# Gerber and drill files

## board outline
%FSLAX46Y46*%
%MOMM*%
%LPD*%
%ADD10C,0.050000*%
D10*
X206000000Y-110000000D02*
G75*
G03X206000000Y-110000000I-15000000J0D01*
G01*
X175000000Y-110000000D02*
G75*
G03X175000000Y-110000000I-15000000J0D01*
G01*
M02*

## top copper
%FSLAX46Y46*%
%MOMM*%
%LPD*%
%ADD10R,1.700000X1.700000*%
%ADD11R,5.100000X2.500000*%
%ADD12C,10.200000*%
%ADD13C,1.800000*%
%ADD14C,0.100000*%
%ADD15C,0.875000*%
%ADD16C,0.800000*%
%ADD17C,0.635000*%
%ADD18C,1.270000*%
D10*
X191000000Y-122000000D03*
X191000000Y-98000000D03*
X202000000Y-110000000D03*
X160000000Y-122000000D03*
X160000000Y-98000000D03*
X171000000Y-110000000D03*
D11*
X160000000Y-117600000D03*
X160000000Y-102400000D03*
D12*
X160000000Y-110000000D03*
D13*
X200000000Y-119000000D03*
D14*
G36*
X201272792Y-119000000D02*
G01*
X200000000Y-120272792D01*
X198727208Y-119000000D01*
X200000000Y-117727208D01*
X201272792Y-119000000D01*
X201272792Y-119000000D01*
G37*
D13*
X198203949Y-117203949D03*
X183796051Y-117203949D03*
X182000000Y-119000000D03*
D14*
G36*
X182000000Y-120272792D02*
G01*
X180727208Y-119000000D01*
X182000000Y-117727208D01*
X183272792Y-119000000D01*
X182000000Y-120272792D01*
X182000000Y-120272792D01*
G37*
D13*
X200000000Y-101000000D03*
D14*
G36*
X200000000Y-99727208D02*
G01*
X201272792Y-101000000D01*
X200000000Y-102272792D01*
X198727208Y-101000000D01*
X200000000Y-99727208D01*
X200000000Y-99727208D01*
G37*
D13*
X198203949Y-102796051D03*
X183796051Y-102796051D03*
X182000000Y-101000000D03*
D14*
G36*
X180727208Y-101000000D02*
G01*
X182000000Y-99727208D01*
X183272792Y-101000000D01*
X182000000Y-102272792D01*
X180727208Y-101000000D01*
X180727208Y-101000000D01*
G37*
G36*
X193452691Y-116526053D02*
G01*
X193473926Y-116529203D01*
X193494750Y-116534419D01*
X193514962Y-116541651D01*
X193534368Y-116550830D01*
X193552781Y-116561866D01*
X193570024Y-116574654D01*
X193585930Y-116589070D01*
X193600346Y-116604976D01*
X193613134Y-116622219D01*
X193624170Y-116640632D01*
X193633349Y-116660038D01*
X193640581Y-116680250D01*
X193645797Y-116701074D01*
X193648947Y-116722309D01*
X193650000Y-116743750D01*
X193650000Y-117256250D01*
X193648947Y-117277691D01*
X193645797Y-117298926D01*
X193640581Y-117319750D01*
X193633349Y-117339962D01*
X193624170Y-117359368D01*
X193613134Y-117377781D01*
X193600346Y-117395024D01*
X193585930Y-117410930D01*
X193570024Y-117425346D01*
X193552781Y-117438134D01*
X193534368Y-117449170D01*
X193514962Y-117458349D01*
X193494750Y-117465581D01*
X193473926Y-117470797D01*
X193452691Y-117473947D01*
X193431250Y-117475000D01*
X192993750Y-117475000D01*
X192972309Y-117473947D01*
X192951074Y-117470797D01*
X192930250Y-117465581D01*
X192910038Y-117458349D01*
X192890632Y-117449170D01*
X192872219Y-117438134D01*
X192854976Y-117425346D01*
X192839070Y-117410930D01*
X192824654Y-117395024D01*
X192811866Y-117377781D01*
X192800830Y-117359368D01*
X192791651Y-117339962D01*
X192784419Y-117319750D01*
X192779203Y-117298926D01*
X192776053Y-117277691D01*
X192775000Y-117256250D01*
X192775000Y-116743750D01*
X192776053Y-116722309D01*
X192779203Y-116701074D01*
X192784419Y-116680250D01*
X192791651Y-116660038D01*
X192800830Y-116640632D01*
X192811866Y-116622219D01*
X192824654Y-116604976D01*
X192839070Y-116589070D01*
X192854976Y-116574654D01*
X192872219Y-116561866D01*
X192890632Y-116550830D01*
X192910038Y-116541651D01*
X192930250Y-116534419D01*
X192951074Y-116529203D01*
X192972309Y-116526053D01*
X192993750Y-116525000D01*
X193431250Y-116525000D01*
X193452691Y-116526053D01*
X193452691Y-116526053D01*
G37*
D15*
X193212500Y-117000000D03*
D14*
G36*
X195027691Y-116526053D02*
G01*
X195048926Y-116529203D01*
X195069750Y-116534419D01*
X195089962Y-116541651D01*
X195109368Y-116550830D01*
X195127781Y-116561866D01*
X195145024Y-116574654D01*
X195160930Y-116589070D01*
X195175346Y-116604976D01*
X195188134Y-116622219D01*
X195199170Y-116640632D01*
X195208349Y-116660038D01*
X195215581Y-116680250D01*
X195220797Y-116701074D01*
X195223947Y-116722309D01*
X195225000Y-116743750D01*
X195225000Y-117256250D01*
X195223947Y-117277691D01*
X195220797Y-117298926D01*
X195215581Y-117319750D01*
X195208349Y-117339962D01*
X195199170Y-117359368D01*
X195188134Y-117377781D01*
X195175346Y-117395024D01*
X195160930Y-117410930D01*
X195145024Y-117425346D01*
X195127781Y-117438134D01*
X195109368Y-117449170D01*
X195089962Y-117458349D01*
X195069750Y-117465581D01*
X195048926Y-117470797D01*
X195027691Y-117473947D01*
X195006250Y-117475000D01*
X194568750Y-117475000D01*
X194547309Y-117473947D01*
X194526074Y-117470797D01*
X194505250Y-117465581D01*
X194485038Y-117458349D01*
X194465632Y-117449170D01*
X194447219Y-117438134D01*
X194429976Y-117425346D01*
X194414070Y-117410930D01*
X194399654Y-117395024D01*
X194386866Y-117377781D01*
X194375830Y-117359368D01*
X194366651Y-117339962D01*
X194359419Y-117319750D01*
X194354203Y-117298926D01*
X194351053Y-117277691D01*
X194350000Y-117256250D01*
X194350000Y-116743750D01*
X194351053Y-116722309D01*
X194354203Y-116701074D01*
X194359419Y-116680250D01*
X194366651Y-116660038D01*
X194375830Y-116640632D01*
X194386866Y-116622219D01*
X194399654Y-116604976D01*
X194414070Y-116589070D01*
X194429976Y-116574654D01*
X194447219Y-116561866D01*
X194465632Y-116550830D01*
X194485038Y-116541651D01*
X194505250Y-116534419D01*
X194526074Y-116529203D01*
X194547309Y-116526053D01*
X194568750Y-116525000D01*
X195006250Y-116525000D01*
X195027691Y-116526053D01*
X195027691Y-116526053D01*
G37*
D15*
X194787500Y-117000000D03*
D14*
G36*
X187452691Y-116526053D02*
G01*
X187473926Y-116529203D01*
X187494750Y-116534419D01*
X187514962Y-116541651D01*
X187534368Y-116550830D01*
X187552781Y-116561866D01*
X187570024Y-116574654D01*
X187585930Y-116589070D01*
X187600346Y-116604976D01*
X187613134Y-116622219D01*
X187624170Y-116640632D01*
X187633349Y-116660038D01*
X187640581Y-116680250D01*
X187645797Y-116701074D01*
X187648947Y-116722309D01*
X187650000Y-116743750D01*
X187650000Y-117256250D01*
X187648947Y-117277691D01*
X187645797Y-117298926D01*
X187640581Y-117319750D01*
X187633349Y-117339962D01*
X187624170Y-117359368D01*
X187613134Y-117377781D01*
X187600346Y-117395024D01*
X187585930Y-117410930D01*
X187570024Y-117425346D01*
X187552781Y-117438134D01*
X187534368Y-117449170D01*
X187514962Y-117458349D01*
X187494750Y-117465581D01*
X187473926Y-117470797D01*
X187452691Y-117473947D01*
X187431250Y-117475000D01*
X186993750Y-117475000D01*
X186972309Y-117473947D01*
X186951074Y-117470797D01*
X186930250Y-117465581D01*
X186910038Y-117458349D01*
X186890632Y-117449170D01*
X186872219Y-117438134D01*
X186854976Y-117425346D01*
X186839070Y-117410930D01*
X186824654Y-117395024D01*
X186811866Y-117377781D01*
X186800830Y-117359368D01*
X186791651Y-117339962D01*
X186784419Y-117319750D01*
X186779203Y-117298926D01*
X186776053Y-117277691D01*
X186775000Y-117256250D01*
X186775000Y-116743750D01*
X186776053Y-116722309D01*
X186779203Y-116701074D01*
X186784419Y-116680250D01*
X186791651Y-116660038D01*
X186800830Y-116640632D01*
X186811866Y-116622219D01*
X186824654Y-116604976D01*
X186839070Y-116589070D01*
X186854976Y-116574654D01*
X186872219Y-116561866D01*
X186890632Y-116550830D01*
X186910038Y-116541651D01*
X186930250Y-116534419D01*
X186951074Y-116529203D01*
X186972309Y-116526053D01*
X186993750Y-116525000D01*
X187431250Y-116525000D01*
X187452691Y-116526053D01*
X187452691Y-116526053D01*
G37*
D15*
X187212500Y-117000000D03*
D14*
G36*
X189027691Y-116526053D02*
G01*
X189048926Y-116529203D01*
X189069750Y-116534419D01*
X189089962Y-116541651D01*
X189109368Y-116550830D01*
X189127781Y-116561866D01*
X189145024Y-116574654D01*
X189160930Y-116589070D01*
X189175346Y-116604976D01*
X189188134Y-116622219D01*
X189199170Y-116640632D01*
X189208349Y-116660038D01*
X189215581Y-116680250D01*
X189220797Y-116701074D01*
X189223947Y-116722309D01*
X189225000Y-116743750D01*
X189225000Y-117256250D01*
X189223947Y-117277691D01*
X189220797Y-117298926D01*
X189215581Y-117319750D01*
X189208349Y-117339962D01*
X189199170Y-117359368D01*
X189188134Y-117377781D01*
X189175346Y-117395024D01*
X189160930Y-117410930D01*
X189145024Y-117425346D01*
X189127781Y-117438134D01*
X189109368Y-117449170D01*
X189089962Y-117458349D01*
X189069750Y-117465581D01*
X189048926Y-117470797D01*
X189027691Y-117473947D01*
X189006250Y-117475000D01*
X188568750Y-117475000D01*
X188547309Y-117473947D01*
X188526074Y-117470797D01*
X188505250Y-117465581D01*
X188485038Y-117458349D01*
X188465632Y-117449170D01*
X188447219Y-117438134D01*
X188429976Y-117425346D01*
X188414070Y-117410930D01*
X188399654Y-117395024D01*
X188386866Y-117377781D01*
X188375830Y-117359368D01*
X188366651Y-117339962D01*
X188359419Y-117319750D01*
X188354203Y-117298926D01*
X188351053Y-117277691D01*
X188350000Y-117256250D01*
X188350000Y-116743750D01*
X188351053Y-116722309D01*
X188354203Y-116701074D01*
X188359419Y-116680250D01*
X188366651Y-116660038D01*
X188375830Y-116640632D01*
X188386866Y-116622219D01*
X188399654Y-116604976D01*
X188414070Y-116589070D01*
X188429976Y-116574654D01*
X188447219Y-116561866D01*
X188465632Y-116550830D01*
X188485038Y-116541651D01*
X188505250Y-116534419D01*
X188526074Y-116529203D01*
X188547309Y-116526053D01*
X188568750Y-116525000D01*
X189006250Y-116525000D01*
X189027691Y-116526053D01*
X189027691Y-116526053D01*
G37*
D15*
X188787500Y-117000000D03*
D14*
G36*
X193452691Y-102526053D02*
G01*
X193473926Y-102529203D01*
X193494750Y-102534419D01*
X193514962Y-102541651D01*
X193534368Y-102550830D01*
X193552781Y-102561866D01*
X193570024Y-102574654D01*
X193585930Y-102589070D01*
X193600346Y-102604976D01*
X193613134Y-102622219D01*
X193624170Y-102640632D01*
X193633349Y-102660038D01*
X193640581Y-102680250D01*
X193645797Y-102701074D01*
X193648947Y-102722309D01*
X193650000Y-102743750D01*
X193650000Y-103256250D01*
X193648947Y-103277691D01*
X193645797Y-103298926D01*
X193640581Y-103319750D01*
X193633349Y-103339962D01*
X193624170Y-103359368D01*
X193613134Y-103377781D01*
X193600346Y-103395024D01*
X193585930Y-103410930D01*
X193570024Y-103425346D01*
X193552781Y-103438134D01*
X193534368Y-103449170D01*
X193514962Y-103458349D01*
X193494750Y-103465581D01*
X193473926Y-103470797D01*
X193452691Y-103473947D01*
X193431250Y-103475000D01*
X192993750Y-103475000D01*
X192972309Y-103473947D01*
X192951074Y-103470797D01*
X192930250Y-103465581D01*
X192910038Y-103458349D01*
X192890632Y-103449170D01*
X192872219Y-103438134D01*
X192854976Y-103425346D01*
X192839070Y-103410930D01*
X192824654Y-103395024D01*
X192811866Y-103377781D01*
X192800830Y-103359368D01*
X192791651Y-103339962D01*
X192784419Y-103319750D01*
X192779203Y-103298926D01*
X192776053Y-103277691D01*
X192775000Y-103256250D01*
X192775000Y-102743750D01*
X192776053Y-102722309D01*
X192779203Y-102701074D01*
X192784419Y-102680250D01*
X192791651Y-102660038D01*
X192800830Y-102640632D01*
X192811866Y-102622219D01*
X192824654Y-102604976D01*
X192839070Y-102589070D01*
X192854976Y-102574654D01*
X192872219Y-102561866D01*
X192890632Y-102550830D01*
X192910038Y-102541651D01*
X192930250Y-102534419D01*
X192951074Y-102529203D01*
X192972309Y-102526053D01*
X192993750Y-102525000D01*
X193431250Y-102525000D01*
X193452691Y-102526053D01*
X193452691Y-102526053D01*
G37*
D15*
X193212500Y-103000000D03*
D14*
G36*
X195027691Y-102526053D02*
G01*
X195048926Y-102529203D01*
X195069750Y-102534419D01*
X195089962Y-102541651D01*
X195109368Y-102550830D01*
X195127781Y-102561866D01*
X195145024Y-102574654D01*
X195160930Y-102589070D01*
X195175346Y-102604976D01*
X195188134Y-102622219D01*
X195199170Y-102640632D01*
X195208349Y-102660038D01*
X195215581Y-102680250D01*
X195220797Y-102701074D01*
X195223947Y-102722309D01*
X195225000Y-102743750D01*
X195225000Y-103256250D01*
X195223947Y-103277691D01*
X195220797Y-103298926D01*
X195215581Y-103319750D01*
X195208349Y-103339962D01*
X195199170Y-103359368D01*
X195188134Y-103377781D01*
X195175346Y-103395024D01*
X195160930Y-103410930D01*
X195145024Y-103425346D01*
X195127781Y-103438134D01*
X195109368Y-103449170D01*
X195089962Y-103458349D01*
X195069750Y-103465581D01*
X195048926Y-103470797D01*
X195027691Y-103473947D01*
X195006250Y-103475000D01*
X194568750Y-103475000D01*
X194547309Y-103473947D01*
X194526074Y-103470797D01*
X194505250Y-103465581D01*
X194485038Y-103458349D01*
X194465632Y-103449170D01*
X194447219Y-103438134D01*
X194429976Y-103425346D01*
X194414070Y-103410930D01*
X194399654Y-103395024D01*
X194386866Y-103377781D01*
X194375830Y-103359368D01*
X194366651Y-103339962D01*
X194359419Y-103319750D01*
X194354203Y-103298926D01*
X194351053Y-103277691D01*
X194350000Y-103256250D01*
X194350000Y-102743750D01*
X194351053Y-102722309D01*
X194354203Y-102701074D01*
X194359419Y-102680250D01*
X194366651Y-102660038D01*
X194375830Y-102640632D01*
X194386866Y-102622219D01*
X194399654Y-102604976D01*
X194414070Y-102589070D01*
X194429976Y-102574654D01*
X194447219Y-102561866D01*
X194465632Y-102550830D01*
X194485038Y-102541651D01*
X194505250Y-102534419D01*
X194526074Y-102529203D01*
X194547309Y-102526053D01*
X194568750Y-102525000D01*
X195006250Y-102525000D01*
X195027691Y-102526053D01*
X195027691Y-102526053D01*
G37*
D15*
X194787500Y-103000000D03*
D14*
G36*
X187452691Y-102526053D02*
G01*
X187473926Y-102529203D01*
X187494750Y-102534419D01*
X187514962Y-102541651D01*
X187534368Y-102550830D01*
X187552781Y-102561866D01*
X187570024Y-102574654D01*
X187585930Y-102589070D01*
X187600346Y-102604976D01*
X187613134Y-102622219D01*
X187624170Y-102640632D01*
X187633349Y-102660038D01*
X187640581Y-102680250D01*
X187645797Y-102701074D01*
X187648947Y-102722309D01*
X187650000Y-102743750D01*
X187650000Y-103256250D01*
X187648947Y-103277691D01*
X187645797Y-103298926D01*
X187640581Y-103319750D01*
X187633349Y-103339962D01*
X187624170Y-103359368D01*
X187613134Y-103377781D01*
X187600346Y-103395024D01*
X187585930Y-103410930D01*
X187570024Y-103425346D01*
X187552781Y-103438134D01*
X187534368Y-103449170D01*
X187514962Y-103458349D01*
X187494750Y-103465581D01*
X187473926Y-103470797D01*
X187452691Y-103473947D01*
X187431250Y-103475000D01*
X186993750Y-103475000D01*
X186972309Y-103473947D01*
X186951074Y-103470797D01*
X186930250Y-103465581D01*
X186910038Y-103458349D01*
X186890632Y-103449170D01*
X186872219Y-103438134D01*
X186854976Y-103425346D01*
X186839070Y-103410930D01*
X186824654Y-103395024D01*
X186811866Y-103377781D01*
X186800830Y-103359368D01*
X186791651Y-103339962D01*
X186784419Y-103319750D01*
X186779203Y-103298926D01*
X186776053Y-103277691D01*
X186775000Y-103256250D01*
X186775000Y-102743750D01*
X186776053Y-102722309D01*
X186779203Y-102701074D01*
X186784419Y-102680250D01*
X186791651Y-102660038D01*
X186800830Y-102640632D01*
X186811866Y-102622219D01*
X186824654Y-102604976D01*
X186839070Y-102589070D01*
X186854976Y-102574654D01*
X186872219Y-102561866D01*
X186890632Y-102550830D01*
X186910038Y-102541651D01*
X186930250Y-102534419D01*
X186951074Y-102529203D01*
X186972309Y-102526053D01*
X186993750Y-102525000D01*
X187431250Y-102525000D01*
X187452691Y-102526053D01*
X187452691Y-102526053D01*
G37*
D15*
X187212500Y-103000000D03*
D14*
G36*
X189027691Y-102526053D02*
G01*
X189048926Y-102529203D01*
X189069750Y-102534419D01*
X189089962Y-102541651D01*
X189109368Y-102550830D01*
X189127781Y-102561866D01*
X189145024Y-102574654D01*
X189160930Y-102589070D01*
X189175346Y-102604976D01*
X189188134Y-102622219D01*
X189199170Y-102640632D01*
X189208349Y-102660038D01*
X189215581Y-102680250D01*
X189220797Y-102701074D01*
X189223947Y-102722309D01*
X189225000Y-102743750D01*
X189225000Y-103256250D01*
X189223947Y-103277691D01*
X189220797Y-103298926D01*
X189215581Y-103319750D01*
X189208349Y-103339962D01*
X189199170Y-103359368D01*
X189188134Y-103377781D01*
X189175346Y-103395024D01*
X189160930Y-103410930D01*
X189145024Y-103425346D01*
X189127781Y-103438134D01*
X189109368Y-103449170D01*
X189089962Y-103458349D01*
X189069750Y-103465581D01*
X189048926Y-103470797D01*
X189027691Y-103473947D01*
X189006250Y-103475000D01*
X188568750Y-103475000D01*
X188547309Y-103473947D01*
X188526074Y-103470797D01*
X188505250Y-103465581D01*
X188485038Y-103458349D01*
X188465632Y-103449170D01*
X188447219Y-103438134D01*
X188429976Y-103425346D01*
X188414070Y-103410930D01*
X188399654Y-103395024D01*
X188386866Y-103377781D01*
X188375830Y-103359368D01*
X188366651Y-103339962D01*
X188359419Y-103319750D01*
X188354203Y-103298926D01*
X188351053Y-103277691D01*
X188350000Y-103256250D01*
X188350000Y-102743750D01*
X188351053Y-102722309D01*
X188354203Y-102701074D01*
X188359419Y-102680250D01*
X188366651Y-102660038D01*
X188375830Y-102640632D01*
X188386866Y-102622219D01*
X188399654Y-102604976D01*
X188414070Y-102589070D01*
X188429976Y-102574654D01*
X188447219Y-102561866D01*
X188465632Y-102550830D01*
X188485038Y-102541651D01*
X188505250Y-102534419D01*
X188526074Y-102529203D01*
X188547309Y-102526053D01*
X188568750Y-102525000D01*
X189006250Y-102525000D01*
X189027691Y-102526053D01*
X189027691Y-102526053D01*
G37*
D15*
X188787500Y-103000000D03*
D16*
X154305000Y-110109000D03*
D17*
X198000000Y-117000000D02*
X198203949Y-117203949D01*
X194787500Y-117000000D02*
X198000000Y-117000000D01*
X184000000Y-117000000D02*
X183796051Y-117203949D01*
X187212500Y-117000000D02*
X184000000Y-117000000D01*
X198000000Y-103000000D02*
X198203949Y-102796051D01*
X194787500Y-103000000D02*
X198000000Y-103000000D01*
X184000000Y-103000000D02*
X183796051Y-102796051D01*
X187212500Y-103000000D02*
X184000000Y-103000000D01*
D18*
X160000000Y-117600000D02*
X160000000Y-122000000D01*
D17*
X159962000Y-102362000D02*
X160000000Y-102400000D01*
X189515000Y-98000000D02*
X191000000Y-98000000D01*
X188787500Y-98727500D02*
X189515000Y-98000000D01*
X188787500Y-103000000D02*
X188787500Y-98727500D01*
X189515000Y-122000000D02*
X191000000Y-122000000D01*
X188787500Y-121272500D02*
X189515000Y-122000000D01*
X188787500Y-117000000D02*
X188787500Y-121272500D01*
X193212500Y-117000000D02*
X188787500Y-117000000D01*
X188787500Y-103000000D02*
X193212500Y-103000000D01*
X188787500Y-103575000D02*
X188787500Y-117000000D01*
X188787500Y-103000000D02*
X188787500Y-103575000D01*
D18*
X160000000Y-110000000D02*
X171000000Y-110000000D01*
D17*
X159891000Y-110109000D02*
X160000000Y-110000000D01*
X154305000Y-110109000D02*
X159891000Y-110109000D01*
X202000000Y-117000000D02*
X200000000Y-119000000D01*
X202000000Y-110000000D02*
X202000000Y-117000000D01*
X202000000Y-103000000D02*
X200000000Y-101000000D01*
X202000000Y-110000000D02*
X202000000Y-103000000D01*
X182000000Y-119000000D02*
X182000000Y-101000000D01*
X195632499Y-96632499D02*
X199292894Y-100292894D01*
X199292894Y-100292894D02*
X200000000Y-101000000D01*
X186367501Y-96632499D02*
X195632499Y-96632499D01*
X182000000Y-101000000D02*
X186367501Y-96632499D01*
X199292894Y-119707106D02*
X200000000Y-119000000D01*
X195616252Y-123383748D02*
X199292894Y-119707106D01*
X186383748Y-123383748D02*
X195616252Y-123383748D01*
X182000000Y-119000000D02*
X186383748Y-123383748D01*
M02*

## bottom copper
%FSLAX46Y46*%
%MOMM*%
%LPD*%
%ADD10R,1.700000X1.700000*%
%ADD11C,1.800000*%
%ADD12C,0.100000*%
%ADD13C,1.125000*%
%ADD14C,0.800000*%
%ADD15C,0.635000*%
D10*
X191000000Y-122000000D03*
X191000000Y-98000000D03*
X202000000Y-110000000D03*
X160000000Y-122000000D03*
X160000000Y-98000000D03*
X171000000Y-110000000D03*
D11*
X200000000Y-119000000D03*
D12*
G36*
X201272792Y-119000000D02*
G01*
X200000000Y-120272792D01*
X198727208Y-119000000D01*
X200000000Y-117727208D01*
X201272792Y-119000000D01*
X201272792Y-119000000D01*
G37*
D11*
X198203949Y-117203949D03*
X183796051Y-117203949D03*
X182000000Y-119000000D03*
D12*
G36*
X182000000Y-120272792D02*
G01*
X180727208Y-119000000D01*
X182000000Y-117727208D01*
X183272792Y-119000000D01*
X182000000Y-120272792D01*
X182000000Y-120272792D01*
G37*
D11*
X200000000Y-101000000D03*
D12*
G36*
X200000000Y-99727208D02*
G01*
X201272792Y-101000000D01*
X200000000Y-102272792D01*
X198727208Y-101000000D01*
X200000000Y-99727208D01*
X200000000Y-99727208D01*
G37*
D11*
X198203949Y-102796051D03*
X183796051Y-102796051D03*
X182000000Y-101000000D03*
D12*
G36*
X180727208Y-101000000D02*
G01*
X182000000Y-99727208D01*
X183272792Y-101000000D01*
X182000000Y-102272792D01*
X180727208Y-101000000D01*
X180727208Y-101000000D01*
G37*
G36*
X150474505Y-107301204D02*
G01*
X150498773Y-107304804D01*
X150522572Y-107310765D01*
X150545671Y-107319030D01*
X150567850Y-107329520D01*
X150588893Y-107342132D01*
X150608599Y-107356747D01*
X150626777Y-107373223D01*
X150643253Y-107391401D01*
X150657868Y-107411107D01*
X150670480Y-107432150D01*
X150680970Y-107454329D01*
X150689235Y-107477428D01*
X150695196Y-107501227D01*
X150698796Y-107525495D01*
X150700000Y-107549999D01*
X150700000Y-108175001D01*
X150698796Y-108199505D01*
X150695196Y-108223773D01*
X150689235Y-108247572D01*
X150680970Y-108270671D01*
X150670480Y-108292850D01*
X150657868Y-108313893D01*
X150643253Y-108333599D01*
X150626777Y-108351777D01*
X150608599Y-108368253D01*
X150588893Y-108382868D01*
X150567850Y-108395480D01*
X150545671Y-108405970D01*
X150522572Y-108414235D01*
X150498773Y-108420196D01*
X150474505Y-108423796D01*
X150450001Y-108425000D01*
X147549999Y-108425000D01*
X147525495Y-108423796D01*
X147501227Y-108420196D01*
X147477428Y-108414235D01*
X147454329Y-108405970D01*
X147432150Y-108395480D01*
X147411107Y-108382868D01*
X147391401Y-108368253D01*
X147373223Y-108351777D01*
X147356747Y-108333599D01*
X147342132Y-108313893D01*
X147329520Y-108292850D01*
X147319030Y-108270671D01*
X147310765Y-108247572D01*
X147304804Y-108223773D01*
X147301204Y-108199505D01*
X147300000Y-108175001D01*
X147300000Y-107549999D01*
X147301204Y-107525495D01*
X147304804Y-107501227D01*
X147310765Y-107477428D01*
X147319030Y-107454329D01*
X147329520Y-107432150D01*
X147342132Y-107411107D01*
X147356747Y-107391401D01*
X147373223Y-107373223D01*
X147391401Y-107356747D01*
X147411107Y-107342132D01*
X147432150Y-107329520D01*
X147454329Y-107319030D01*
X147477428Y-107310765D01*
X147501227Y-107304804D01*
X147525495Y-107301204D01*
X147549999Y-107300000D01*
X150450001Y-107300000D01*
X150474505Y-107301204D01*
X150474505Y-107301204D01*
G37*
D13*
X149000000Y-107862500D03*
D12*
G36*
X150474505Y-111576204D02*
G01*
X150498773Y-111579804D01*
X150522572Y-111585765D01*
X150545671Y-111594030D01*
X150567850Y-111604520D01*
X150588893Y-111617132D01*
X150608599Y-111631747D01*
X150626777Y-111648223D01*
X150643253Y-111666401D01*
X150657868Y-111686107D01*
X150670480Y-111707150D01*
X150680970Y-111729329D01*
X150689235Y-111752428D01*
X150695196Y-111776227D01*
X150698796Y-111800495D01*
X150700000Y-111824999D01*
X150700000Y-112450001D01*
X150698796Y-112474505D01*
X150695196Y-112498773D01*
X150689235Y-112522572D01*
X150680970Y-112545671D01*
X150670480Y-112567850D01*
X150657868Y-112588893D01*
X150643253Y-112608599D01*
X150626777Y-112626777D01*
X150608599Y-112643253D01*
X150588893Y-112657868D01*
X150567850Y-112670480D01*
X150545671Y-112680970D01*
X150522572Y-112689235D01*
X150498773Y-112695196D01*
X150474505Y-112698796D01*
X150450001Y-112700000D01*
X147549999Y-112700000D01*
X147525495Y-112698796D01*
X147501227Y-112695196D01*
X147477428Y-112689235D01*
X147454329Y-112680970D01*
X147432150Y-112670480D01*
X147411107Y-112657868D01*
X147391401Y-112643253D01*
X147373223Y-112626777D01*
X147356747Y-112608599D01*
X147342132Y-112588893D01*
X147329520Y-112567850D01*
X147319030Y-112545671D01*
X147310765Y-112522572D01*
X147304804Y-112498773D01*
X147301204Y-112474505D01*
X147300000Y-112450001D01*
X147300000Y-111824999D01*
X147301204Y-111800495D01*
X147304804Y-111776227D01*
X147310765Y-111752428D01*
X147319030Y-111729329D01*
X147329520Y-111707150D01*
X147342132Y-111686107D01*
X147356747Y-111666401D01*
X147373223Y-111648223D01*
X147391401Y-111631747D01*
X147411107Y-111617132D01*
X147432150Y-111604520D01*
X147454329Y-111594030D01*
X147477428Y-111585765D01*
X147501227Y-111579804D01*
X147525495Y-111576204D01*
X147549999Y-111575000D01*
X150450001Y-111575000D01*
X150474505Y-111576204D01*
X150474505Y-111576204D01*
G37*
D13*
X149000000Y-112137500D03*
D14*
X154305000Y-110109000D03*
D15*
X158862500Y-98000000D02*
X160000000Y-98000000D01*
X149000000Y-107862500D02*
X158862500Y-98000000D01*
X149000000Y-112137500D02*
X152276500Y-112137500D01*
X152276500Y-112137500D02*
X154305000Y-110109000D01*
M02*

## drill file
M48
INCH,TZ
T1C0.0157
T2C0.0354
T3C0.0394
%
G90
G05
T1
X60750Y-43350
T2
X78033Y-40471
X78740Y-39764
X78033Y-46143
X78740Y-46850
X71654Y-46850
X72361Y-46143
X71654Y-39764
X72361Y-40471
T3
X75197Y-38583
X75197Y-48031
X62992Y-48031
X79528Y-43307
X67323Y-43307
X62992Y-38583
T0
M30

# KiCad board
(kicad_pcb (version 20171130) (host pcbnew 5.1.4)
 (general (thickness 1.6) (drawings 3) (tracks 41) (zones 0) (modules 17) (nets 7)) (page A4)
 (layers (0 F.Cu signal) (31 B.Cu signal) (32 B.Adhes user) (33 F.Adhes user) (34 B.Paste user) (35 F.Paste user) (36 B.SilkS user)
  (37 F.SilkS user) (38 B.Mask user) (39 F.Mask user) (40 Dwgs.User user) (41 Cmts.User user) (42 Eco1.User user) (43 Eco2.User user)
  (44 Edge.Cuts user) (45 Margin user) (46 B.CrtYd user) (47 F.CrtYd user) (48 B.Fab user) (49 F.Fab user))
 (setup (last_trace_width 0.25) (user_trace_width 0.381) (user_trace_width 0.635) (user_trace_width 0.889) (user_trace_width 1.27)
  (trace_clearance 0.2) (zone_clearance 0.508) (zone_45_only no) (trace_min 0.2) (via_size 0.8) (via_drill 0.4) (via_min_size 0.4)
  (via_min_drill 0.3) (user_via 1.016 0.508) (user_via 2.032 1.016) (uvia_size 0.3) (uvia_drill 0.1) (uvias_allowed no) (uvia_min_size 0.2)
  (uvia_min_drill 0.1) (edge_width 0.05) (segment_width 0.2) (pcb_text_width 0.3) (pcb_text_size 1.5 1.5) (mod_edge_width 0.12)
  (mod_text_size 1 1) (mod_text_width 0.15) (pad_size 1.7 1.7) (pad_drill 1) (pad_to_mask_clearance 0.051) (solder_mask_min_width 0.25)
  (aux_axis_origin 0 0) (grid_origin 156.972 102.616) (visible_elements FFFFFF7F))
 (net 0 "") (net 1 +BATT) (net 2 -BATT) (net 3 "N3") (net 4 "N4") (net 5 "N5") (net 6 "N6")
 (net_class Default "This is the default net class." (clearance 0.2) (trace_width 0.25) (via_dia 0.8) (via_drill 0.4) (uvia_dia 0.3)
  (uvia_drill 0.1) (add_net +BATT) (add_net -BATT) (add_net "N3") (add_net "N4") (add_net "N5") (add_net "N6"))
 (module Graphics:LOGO (layer B.Cu) (at 184.785 116.205)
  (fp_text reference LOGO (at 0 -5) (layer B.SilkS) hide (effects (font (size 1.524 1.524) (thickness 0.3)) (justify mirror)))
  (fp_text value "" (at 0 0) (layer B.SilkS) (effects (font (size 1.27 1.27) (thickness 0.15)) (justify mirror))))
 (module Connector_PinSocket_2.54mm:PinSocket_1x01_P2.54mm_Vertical (layer F.Cu) (at 191 122)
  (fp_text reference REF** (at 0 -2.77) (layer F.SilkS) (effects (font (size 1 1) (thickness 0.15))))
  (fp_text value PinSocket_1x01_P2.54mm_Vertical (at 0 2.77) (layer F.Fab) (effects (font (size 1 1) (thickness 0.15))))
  (pad 1 thru_hole rect (at 0 0) (size 1.7 1.7) (drill 1) (layers *.Cu *.Mask) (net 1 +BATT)))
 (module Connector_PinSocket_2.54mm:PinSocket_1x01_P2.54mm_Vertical (layer F.Cu) (at 191 98)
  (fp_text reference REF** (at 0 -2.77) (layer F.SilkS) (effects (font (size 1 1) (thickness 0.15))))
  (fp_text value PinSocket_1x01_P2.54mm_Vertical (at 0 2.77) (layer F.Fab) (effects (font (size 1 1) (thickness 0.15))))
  (pad 1 thru_hole rect (at 0 0) (size 1.7 1.7) (drill 1) (layers *.Cu *.Mask) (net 1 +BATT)))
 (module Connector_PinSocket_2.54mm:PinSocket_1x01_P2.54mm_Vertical (layer F.Cu) (at 202 110)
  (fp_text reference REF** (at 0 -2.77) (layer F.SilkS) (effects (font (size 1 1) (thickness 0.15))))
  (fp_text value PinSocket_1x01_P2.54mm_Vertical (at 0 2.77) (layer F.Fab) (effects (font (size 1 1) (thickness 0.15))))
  (pad 1 thru_hole rect (at 0 0) (size 1.7 1.7) (drill 1) (layers *.Cu *.Mask) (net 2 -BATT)))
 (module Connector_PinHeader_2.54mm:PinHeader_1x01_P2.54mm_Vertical (layer F.Cu) (at 160 122 180)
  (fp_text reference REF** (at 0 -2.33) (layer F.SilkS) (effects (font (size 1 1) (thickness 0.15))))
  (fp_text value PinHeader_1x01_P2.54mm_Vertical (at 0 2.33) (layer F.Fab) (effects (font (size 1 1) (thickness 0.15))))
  (pad 1 thru_hole rect (at 0 0 180) (size 1.7 1.7) (drill 1) (layers *.Cu *.Mask) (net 1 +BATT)))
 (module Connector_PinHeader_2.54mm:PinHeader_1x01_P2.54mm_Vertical (layer F.Cu) (at 160 98)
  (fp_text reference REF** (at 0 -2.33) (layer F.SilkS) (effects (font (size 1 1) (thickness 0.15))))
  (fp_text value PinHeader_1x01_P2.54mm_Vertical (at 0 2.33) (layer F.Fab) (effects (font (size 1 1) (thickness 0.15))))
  (pad 1 thru_hole rect (at 0 0) (size 1.7 1.7) (drill 1) (layers *.Cu *.Mask) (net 1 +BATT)))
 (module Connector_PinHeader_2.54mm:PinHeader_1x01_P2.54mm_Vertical (layer F.Cu) (at 171 110 90)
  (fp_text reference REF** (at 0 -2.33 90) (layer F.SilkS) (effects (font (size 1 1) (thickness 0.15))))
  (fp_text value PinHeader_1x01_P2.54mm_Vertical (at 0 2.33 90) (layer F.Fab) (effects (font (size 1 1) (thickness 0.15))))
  (pad 1 thru_hole rect (at 0 0 90) (size 1.7 1.7) (drill 1) (layers *.Cu *.Mask) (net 2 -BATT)))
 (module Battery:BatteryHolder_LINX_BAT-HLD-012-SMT (layer F.Cu) (at 160 110 90)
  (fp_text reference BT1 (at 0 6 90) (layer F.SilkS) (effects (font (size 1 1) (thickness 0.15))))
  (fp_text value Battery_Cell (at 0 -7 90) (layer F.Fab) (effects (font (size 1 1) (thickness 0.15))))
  (pad 1 smd rect (at -7.6 0 90) (size 2.5 5.1) (layers F.Cu F.Paste F.Mask) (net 1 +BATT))
  (pad 1 smd rect (at 7.6 0 90) (size 2.5 5.1) (layers F.Cu F.Paste F.Mask) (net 1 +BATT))
  (pad 2 smd circle (at 0 0 90) (size 10.2 10.2) (layers F.Cu F.Paste F.Mask) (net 2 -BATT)))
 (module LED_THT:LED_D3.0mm (layer F.Cu) (at 200 119 135)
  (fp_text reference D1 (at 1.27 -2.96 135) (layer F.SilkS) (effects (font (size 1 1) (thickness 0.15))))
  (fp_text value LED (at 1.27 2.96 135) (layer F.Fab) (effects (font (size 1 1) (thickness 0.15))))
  (pad 1 thru_hole rect (at 0 0 135) (size 1.8 1.8) (drill 0.9) (layers *.Cu *.Mask) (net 2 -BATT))
  (pad 2 thru_hole circle (at 2.54 0 135) (size 1.8 1.8) (drill 0.9) (layers *.Cu *.Mask) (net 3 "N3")))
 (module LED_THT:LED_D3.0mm (layer F.Cu) (at 182 119 45)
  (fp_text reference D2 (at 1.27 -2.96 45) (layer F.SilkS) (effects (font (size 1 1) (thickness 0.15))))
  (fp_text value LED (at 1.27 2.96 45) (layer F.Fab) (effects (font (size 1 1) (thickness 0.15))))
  (pad 2 thru_hole circle (at 2.54 0 45) (size 1.8 1.8) (drill 0.9) (layers *.Cu *.Mask) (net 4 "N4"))
  (pad 1 thru_hole rect (at 0 0 45) (size 1.8 1.8) (drill 0.9) (layers *.Cu *.Mask) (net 2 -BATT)))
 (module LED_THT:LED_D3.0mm (layer F.Cu) (at 200 101 225)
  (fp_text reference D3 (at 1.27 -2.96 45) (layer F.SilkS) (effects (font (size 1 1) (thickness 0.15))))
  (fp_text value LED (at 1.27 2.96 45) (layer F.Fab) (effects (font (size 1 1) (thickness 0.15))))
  (pad 1 thru_hole rect (at 0 0 225) (size 1.8 1.8) (drill 0.9) (layers *.Cu *.Mask) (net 2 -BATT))
  (pad 2 thru_hole circle (at 2.54 0 225) (size 1.8 1.8) (drill 0.9) (layers *.Cu *.Mask) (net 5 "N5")))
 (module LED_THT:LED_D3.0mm (layer F.Cu) (at 182 101 315)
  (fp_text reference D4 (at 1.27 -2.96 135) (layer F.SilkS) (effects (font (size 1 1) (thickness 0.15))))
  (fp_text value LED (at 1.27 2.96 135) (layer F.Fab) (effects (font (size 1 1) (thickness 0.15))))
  (pad 2 thru_hole circle (at 2.54 0 315) (size 1.8 1.8) (drill 0.9) (layers *.Cu *.Mask) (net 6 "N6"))
  (pad 1 thru_hole rect (at 0 0 315) (size 1.8 1.8) (drill 0.9) (layers *.Cu *.Mask) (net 2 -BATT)))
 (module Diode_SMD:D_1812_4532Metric (layer B.Cu) (at 149 110 270)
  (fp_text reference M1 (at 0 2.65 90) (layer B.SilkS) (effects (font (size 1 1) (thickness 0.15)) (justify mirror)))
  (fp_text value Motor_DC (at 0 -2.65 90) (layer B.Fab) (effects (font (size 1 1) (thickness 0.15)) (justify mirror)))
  (pad 1 smd roundrect (at -2.1375 0 270) (size 1.125 3.4) (layers B.Cu B.Paste B.Mask) (roundrect_rratio 0.222222) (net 1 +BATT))
  (pad 2 smd roundrect (at 2.1375 0 270) (size 1.125 3.4) (layers B.Cu B.Paste B.Mask) (roundrect_rratio 0.222222) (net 2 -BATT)))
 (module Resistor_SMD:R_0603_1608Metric (layer F.Cu) (at 194 117)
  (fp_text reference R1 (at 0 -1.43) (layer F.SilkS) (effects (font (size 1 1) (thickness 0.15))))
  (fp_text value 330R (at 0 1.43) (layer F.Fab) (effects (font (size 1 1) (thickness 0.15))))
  (pad 1 smd roundrect (at -0.7875 0) (size 0.875 0.95) (layers F.Cu F.Paste F.Mask) (roundrect_rratio 0.25) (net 1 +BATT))
  (pad 2 smd roundrect (at 0.7875 0) (size 0.875 0.95) (layers F.Cu F.Paste F.Mask) (roundrect_rratio 0.25) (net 3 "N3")))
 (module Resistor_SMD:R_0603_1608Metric (layer F.Cu) (at 188 117 180)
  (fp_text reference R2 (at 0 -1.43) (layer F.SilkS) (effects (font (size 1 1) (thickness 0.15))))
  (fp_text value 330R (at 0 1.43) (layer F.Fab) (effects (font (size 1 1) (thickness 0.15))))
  (pad 2 smd roundrect (at 0.7875 0 180) (size 0.875 0.95) (layers F.Cu F.Paste F.Mask) (roundrect_rratio 0.25) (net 4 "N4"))
  (pad 1 smd roundrect (at -0.7875 0 180) (size 0.875 0.95) (layers F.Cu F.Paste F.Mask) (roundrect_rratio 0.25) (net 1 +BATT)))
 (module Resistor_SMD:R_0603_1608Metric (layer F.Cu) (at 194 103)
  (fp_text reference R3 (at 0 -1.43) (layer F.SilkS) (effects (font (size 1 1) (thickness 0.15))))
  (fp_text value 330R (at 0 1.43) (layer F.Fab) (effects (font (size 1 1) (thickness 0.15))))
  (pad 1 smd roundrect (at -0.7875 0) (size 0.875 0.95) (layers F.Cu F.Paste F.Mask) (roundrect_rratio 0.25) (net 1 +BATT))
  (pad 2 smd roundrect (at 0.7875 0) (size 0.875 0.95) (layers F.Cu F.Paste F.Mask) (roundrect_rratio 0.25) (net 5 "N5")))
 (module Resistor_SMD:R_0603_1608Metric (layer F.Cu) (at 188 103 180)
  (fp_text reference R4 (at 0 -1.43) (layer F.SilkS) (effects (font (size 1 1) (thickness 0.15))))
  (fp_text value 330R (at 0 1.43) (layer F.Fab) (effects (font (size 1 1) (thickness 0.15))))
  (pad 2 smd roundrect (at 0.7875 0 180) (size 0.875 0.95) (layers F.Cu F.Paste F.Mask) (roundrect_rratio 0.25) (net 6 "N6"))
  (pad 1 smd roundrect (at -0.7875 0 180) (size 0.875 0.95) (layers F.Cu F.Paste F.Mask) (roundrect_rratio 0.25) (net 1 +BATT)))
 (gr_circle (center 191 110) (end 176 110) (layer Edge.Cuts) (width 0.05))
 (gr_circle (center 160 110) (end 175 110) (layer Edge.Cuts) (width 0.05))
 (segment (start 198 117) (end 198.203949 117.203949) (width 0.635) (layer F.Cu) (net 3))
 (segment (start 194.7875 117) (end 198 117) (width 0.635) (layer F.Cu) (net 3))
 (segment (start 184 117) (end 183.796051 117.203949) (width 0.635) (layer F.Cu) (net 4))
 (segment (start 187.2125 117) (end 184 117) (width 0.635) (layer F.Cu) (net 4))
 (segment (start 198 103) (end 198.203949 102.796051) (width 0.635) (layer F.Cu) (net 5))
 (segment (start 194.7875 103) (end 198 103) (width 0.635) (layer F.Cu) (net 5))
 (segment (start 184 103) (end 183.796051 102.796051) (width 0.635) (layer F.Cu) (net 6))
 (segment (start 187.2125 103) (end 184 103) (width 0.635) (layer F.Cu) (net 6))
 (segment (start 160 117.6) (end 160 122) (width 1.27) (layer F.Cu) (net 1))
 (segment (start 159.962 102.362) (end 160 102.4) (width 0.635) (layer F.Cu) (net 1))
 (segment (start 189.515 98) (end 191 98) (width 0.635) (layer F.Cu) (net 1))
 (segment (start 188.7875 98.7275) (end 189.515 98) (width 0.635) (layer F.Cu) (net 1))
 (segment (start 188.7875 103) (end 188.7875 98.7275) (width 0.635) (layer F.Cu) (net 1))
 (segment (start 189.515 122) (end 191 122) (width 0.635) (layer F.Cu) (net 1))
 (segment (start 188.7875 121.2725) (end 189.515 122) (width 0.635) (layer F.Cu) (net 1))
 (segment (start 188.7875 117) (end 188.7875 121.2725) (width 0.635) (layer F.Cu) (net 1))
 (segment (start 193.2125 117) (end 188.7875 117) (width 0.635) (layer F.Cu) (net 1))
 (segment (start 188.7875 103) (end 193.2125 103) (width 0.635) (layer F.Cu) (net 1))
 (segment (start 188.7875 103.575) (end 188.7875 117) (width 0.635) (layer F.Cu) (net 1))
 (segment (start 188.7875 103) (end 188.7875 103.575) (width 0.635) (layer F.Cu) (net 1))
 (segment (start 158.8625 98) (end 160 98) (width 0.635) (layer B.Cu) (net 1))
 (segment (start 149 107.8625) (end 158.8625 98) (width 0.635) (layer B.Cu) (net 1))
 (segment (start 160 110) (end 171 110) (width 1.27) (layer F.Cu) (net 2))
 (via (at 154.305 110.109) (size 0.8) (drill 0.4) (layers F.Cu B.Cu) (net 2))
 (segment (start 149 112.1375) (end 152.2765 112.1375) (width 0.635) (layer B.Cu) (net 2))
 (segment (start 152.2765 112.1375) (end 154.305 110.109) (width 0.635) (layer B.Cu) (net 2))
 (segment (start 159.891 110.109) (end 160 110) (width 0.635) (layer F.Cu) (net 2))
 (segment (start 154.305 110.109) (end 159.891 110.109) (width 0.635) (layer F.Cu) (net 2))
 (segment (start 202 117) (end 200 119) (width 0.635) (layer F.Cu) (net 2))
 (segment (start 202 110) (end 202 117) (width 0.635) (layer F.Cu) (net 2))
 (segment (start 202 103) (end 200 101) (width 0.635) (layer F.Cu) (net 2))
 (segment (start 202 110) (end 202 103) (width 0.635) (layer F.Cu) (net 2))
 (segment (start 182 119) (end 182 101) (width 0.635) (layer F.Cu) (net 2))
 (segment (start 195.632499 96.632499) (end 199.292894 100.292894) (width 0.635) (layer F.Cu) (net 2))
 (segment (start 199.292894 100.292894) (end 200 101) (width 0.635) (layer F.Cu) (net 2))
 (segment (start 186.367501 96.632499) (end 195.632499 96.632499) (width 0.635) (layer F.Cu) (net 2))
 (segment (start 182 101) (end 186.367501 96.632499) (width 0.635) (layer F.Cu) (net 2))
 (segment (start 199.292894 119.707106) (end 200 119) (width 0.635) (layer F.Cu) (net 2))
 (segment (start 195.616252 123.383748) (end 199.292894 119.707106) (width 0.635) (layer F.Cu) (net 2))
 (segment (start 186.383748 123.383748) (end 195.616252 123.383748) (width 0.635) (layer F.Cu) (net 2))
 (segment (start 182 119) (end 186.383748 123.383748) (width 0.635) (layer F.Cu) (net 2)))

